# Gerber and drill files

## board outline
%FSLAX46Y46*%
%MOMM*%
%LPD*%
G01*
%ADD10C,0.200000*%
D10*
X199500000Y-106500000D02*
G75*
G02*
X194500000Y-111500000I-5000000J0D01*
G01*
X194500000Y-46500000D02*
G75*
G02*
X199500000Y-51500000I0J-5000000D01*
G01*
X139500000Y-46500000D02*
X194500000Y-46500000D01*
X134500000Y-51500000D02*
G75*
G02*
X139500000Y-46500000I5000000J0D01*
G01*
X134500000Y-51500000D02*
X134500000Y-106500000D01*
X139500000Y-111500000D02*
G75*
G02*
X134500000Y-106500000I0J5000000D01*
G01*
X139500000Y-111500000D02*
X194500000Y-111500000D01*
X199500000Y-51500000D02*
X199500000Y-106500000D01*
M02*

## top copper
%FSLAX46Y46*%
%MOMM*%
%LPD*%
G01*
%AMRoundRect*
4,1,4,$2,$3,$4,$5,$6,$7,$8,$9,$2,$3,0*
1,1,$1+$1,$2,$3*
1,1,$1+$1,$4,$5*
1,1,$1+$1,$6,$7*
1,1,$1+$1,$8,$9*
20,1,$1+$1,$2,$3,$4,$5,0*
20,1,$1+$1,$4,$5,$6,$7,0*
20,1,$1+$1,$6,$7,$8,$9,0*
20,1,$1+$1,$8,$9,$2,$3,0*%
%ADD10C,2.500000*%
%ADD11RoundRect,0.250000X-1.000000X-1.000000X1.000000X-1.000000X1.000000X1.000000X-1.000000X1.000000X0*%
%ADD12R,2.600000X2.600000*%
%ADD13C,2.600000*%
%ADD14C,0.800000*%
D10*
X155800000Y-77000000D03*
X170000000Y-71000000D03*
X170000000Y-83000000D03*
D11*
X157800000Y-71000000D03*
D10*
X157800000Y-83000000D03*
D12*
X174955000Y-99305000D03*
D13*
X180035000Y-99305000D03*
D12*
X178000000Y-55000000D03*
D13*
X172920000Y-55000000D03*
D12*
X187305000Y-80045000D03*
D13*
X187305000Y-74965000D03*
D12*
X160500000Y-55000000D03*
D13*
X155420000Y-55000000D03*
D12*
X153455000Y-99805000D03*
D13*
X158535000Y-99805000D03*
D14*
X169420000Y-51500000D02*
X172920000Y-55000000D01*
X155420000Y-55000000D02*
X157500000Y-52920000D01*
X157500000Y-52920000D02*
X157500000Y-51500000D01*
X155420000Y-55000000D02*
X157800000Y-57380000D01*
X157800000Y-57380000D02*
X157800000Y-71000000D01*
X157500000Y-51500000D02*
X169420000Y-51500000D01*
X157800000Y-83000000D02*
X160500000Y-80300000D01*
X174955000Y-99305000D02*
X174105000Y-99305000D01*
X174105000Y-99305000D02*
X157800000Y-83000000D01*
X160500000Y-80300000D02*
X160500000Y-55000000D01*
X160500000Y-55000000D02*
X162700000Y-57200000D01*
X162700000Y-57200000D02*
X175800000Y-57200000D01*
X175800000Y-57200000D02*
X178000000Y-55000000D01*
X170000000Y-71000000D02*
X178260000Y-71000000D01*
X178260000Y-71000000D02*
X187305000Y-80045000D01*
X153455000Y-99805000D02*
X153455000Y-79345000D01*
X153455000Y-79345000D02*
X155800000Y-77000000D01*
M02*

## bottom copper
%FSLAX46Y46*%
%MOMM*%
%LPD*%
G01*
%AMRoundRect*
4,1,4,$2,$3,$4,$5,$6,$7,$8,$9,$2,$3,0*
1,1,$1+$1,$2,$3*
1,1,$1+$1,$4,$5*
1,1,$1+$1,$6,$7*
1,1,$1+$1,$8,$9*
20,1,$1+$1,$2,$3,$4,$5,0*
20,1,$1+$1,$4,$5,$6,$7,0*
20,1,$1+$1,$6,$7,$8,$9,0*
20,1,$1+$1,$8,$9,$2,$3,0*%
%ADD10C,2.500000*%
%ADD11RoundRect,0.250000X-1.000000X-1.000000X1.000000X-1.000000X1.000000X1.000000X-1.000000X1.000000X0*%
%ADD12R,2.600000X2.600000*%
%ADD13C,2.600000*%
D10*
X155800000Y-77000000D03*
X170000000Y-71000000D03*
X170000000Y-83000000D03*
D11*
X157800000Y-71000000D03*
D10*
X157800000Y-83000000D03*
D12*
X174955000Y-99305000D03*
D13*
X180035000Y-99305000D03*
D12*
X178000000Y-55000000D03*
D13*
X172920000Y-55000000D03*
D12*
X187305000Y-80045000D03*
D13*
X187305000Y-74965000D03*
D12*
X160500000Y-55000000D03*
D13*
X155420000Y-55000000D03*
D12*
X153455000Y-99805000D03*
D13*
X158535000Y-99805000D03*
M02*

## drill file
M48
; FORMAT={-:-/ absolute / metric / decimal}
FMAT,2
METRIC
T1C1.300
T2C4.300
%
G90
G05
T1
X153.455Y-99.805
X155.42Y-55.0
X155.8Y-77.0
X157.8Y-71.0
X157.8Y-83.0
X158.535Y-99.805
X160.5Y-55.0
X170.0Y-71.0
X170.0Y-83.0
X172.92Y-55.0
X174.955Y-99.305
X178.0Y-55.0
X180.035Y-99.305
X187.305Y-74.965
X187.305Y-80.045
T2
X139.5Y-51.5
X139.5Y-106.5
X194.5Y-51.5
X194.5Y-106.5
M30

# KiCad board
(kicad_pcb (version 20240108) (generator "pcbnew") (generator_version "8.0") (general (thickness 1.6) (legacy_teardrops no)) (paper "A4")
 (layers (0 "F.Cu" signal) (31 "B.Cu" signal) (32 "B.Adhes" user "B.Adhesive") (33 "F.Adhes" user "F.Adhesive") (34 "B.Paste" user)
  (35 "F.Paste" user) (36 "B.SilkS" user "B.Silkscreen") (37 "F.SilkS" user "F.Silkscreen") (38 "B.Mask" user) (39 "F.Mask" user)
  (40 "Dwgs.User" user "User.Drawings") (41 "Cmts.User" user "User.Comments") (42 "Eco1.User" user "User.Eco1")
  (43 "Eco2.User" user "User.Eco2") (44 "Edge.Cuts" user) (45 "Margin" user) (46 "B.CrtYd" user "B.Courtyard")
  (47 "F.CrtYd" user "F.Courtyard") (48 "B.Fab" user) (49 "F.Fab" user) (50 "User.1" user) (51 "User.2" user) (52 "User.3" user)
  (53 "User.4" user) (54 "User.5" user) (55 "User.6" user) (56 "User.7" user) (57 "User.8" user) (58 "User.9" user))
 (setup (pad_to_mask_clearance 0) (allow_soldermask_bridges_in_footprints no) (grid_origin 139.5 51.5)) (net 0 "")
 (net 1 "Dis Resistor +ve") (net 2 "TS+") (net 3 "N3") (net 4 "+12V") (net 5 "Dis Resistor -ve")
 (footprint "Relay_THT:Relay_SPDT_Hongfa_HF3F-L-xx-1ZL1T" (layer "F.Cu") (at 157.8 71)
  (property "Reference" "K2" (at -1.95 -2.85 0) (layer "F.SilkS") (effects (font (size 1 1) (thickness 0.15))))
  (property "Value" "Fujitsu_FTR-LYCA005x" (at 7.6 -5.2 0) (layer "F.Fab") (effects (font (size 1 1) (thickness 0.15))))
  (pad "11" thru_hole circle (at -2 6) (size 2.5 2.5) (drill 1.3) (layers "*.Cu" "*.Mask") (remove_unused_layers no)
   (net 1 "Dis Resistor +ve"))
  (pad "12" thru_hole circle (at 12.2 0) (size 2.5 2.5) (drill 1.3) (layers "*.Cu" "*.Mask") (remove_unused_layers no) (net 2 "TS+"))
  (pad "14" thru_hole circle (at 12.2 12) (size 2.5 2.5) (drill 1.3) (layers "*.Cu" "*.Mask") (remove_unused_layers no) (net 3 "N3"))
  (pad "A1" thru_hole roundrect (at 0 0) (size 2.5 2.5) (drill 1.3) (layers "*.Cu" "*.Mask") (remove_unused_layers no)
   (roundrect_rratio 0.1) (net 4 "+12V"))
  (pad "A2" thru_hole circle (at 0 12) (size 2.5 2.5) (drill 1.3) (layers "*.Cu" "*.Mask") (remove_unused_layers no)
   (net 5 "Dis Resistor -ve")))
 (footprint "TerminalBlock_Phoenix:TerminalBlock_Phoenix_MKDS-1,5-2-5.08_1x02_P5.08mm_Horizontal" (layer "F.Cu") (at 174.955 99.305)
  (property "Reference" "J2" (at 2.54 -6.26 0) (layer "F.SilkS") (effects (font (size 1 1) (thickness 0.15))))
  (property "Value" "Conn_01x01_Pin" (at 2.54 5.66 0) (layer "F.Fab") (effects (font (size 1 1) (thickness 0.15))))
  (pad "1" thru_hole rect (at 0 0) (size 2.6 2.6) (drill 1.3) (layers "*.Cu" "*.Mask") (remove_unused_layers no) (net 5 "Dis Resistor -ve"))
  (pad "2" thru_hole circle (at 5.08 0) (size 2.6 2.6) (drill 1.3) (layers "*.Cu" "*.Mask") (remove_unused_layers no)))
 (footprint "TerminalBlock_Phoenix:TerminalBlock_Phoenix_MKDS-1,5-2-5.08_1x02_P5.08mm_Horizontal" (layer "F.Cu") (at 178 55 180)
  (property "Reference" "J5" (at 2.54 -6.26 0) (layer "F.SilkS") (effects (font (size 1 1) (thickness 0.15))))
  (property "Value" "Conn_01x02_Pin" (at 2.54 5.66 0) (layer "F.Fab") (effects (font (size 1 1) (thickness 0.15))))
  (pad "1" thru_hole rect (at 0 0 180) (size 2.6 2.6) (drill 1.3) (layers "*.Cu" "*.Mask") (remove_unused_layers no)
   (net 5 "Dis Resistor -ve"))
  (pad "2" thru_hole circle (at 5.08 0 180) (size 2.6 2.6) (drill 1.3) (layers "*.Cu" "*.Mask") (remove_unused_layers no) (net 4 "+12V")))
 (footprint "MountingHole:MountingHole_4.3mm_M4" (layer "F.Cu") (at 139.5 51.5)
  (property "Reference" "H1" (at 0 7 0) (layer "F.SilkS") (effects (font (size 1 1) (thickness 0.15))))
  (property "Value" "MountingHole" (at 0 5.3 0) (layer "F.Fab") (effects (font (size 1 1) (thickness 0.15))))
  (pad "" np_thru_hole circle (at 0 0) (size 4.3 4.3) (drill 4.3) (layers "*.Cu" "*.Mask")))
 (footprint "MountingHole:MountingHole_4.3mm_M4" (layer "F.Cu") (at 139.5 106.5)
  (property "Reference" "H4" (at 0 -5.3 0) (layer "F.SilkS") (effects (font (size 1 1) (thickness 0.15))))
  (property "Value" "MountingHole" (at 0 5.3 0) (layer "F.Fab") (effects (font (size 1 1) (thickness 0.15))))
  (pad "" np_thru_hole circle (at 0 0) (size 4.3 4.3) (drill 4.3) (layers "*.Cu" "*.Mask")))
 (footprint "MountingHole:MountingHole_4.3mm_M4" (layer "F.Cu") (at 194.5 106.5)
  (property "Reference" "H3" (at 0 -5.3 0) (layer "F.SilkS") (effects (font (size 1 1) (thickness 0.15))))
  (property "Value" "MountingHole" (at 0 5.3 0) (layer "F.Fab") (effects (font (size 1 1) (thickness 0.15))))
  (pad "" np_thru_hole circle (at 0 0) (size 4.3 4.3) (drill 4.3) (layers "*.Cu" "*.Mask")))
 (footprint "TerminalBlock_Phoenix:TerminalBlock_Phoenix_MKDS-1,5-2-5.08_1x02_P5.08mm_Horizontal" (layer "F.Cu") (at 187.305 80.045 90)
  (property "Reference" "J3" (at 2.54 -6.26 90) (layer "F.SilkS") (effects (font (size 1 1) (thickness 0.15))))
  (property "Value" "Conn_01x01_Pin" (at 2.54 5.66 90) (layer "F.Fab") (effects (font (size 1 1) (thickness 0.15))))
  (pad "1" thru_hole rect (at 0 0 90) (size 2.6 2.6) (drill 1.3) (layers "*.Cu" "*.Mask") (remove_unused_layers no) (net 2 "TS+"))
  (pad "2" thru_hole circle (at 5.08 0 90) (size 2.6 2.6) (drill 1.3) (layers "*.Cu" "*.Mask") (remove_unused_layers no)))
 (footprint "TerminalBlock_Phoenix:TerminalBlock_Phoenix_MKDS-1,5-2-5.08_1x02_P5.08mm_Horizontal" (layer "F.Cu") (at 160.5 55 180)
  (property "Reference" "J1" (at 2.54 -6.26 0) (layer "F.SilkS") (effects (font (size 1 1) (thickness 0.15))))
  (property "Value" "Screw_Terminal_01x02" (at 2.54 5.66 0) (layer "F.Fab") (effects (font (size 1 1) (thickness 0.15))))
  (pad "1" thru_hole rect (at 0 0 180) (size 2.6 2.6) (drill 1.3) (layers "*.Cu" "*.Mask") (remove_unused_layers no)
   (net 5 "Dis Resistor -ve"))
  (pad "2" thru_hole circle (at 5.08 0 180) (size 2.6 2.6) (drill 1.3) (layers "*.Cu" "*.Mask") (remove_unused_layers no) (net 4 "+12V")))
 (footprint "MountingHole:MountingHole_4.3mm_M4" (layer "F.Cu") (at 194.5 51.5)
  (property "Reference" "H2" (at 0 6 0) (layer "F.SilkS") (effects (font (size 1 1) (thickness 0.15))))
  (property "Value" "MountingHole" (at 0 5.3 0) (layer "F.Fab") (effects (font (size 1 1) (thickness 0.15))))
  (pad "" np_thru_hole circle (at 0 0) (size 4.3 4.3) (drill 4.3) (layers "*.Cu" "*.Mask")))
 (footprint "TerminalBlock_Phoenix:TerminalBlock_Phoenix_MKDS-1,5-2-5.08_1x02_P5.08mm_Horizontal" (layer "F.Cu") (at 153.455 99.805)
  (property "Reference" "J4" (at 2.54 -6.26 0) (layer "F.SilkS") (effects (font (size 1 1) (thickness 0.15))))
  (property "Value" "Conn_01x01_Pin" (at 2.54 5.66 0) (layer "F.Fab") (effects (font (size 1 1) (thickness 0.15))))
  (pad "1" thru_hole rect (at 0 0) (size 2.6 2.6) (drill 1.3) (layers "*.Cu" "*.Mask") (remove_unused_layers no) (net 1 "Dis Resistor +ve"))
  (pad "2" thru_hole circle (at 5.08 0) (size 2.6 2.6) (drill 1.3) (layers "*.Cu" "*.Mask") (remove_unused_layers no)))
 (gr_arc (start 199.5 106.5) (mid 198.035534 110.035534) (end 194.5 111.5) (stroke (width 0.2) (type default)) (layer "Edge.Cuts"))
 (gr_arc (start 194.5 46.5) (mid 198.035534 47.964466) (end 199.5 51.5) (stroke (width 0.2) (type default)) (layer "Edge.Cuts"))
 (gr_line (start 139.5 46.5) (end 194.5 46.5) (stroke (width 0.2) (type default)) (layer "Edge.Cuts"))
 (gr_arc (start 134.5 51.5) (mid 135.964466 47.964466) (end 139.5 46.5) (stroke (width 0.2) (type default)) (layer "Edge.Cuts"))
 (gr_line (start 134.5 51.5) (end 134.5 106.5) (stroke (width 0.2) (type default)) (layer "Edge.Cuts"))
 (gr_arc (start 139.5 111.5) (mid 135.964466 110.035534) (end 134.5 106.5) (stroke (width 0.2) (type default)) (layer "Edge.Cuts"))
 (gr_line (start 139.5 111.5) (end 194.5 111.5) (stroke (width 0.2) (type default)) (layer "Edge.Cuts"))
 (gr_line (start 199.5 51.5) (end 199.5 106.5) (stroke (width 0.2) (type default)) (layer "Edge.Cuts"))
 (segment (start 169.42 51.5) (end 172.92 55) (width 0.8) (layer "F.Cu") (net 4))
 (segment (start 155.42 55) (end 157.5 52.92) (width 0.8) (layer "F.Cu") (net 4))
 (segment (start 157.5 52.92) (end 157.5 51.5) (width 0.8) (layer "F.Cu") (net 4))
 (segment (start 155.42 55) (end 157.8 57.38) (width 0.8) (layer "F.Cu") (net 4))
 (segment (start 157.8 57.38) (end 157.8 71) (width 0.8) (layer "F.Cu") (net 4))
 (segment (start 157.5 51.5) (end 169.42 51.5) (width 0.8) (layer "F.Cu") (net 4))
 (segment (start 157.8 83) (end 160.5 80.3) (width 0.8) (layer "F.Cu") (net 5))
 (segment (start 174.955 99.305) (end 174.105 99.305) (width 0.8) (layer "F.Cu") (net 5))
 (segment (start 174.105 99.305) (end 157.8 83) (width 0.8) (layer "F.Cu") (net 5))
 (segment (start 160.5 80.3) (end 160.5 55) (width 0.8) (layer "F.Cu") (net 5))
 (segment (start 160.5 55) (end 162.7 57.2) (width 0.8) (layer "F.Cu") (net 5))
 (segment (start 162.7 57.2) (end 175.8 57.2) (width 0.8) (layer "F.Cu") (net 5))
 (segment (start 175.8 57.2) (end 178 55) (width 0.8) (layer "F.Cu") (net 5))
 (segment (start 170 71) (end 178.26 71) (width 0.8) (layer "F.Cu") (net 2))
 (segment (start 178.26 71) (end 187.305 80.045) (width 0.8) (layer "F.Cu") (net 2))
 (segment (start 153.455 99.805) (end 153.455 79.345) (width 0.8) (layer "F.Cu") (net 1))
 (segment (start 153.455 79.345) (end 155.8 77) (width 0.8) (layer "F.Cu") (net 1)))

